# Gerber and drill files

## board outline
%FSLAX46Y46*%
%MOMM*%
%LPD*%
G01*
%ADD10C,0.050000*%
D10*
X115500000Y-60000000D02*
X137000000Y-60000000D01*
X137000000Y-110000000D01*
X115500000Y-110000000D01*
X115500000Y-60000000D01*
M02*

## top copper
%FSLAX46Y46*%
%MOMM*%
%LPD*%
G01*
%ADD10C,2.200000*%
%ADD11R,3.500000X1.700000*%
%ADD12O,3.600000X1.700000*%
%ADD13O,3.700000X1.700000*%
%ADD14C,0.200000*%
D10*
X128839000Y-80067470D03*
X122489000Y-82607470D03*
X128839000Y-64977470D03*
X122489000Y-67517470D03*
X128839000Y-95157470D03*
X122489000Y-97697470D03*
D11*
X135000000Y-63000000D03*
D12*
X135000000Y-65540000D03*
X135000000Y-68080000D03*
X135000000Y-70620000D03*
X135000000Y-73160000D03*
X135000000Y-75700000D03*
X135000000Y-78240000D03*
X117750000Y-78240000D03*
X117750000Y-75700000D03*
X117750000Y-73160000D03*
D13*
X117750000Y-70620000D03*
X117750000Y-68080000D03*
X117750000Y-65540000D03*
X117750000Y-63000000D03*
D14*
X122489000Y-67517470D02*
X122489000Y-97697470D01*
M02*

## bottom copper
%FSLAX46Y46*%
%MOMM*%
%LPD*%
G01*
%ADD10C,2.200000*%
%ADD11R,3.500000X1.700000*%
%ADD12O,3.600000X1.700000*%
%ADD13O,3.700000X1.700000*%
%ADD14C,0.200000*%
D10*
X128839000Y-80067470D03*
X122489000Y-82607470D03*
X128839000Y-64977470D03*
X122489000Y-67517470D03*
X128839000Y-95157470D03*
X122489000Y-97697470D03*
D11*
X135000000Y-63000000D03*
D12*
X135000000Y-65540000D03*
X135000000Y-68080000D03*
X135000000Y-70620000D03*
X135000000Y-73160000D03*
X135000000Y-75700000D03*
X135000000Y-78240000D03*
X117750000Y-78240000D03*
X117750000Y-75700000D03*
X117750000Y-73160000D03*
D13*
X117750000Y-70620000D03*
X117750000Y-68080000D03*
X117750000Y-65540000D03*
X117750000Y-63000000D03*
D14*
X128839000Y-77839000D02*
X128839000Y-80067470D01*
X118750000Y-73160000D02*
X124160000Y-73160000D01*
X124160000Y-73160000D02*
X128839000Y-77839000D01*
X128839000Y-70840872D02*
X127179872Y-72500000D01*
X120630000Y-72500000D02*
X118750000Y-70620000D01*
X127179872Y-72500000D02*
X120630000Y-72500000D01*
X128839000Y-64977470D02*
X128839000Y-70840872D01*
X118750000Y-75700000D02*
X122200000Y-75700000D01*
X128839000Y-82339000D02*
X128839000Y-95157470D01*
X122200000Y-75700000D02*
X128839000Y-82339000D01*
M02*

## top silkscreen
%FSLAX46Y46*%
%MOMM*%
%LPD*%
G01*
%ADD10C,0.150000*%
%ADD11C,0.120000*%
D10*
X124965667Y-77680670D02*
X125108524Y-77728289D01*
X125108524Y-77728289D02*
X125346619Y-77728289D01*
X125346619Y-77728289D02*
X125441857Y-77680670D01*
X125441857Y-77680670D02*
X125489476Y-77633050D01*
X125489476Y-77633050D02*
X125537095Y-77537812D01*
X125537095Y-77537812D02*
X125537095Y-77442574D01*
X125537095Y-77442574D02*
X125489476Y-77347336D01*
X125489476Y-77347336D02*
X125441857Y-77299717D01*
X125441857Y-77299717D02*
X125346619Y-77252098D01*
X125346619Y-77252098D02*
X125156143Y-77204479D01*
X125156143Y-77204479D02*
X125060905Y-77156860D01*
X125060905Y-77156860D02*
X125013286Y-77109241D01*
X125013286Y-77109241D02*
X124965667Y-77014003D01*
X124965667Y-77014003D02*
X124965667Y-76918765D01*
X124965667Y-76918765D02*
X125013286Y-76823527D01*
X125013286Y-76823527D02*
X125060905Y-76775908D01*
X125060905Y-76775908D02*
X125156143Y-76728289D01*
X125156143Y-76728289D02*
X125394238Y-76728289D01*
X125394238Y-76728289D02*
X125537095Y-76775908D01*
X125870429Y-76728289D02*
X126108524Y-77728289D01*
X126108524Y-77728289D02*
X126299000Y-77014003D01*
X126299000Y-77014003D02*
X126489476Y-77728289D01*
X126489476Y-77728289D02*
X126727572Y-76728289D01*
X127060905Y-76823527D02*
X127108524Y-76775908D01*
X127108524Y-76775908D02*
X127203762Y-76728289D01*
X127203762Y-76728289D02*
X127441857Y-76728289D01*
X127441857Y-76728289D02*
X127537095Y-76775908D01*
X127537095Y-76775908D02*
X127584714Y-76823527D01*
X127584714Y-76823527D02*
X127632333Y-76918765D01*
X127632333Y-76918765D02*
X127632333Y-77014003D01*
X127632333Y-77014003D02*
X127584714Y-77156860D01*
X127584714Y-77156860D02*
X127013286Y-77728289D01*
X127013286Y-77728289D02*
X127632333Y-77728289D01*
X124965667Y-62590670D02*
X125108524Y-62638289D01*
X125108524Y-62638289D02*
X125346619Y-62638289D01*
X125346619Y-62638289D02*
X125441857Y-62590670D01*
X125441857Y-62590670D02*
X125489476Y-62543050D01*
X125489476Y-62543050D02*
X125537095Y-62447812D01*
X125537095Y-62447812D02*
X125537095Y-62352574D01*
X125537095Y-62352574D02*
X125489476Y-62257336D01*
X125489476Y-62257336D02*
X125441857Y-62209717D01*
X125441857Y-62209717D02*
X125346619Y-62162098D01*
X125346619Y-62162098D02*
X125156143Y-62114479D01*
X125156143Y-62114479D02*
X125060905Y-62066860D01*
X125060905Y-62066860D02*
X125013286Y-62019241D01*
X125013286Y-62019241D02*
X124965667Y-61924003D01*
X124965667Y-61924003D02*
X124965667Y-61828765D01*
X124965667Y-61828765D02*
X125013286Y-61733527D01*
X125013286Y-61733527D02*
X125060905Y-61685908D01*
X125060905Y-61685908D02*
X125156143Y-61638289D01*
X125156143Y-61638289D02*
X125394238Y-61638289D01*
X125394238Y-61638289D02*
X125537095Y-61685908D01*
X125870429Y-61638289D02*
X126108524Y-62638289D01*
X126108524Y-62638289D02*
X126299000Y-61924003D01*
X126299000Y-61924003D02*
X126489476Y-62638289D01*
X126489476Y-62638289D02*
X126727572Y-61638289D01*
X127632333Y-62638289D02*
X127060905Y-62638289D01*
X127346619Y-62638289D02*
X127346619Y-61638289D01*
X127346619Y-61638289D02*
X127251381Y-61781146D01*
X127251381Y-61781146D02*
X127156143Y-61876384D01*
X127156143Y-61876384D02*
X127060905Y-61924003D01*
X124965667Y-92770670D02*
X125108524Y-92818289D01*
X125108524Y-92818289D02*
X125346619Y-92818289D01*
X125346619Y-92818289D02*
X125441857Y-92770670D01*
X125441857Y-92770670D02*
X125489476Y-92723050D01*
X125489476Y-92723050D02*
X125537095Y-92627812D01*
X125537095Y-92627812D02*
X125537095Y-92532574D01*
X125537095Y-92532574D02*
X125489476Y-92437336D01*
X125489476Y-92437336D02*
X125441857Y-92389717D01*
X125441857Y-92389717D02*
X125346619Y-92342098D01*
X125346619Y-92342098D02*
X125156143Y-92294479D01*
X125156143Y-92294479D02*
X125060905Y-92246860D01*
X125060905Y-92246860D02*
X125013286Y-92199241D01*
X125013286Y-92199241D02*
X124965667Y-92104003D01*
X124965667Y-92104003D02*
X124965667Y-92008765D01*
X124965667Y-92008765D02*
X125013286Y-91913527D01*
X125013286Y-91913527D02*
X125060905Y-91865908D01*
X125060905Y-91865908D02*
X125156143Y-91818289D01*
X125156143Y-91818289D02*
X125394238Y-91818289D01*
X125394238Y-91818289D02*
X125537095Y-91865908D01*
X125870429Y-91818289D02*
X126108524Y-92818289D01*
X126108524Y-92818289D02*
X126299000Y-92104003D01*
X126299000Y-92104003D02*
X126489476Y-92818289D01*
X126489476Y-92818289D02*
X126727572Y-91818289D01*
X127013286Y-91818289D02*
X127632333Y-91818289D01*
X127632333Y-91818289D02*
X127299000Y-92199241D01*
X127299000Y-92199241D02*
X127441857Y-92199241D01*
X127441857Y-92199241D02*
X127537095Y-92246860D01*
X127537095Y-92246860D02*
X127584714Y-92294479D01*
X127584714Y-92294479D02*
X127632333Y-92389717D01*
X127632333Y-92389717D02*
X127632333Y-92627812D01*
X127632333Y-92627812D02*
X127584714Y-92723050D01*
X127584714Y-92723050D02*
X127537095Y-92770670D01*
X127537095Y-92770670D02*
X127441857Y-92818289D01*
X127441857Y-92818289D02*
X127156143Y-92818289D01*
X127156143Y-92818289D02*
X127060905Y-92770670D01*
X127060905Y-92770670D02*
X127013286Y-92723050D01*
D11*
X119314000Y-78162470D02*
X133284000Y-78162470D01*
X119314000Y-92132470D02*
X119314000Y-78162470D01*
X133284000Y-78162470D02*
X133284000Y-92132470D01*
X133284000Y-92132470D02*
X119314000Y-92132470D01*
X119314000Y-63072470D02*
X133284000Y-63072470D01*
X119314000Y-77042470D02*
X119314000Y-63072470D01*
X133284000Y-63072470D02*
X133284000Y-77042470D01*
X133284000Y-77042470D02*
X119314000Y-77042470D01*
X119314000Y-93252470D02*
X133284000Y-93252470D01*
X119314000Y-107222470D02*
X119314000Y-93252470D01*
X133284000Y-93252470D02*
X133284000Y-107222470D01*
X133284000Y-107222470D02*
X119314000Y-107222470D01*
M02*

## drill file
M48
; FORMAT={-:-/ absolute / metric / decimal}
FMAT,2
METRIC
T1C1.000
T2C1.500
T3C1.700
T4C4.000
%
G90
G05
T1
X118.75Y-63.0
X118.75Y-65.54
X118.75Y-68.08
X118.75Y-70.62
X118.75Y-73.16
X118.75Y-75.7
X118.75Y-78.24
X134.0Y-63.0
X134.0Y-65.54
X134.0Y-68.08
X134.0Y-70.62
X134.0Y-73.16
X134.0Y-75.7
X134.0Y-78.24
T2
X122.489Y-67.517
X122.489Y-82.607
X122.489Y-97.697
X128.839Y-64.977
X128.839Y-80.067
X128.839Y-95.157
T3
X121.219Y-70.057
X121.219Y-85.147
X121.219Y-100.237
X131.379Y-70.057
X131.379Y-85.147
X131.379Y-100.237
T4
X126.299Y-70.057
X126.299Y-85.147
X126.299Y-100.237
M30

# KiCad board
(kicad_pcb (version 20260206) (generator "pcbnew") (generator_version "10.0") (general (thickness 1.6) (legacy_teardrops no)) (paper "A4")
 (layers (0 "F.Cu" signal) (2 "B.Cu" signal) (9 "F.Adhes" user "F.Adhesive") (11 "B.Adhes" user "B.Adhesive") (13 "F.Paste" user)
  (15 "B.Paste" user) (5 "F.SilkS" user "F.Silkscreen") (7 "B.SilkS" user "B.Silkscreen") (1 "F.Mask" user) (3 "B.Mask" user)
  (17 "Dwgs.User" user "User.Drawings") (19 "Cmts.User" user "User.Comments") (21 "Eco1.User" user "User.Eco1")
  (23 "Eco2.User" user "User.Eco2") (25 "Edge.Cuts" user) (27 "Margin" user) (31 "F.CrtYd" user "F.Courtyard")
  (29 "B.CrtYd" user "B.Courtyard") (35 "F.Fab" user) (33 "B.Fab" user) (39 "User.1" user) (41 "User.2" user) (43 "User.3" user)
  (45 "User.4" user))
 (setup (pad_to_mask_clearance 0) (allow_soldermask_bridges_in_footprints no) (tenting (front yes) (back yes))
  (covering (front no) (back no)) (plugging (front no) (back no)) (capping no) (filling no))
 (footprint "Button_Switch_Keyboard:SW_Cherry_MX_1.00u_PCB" (layer "F.Cu") (at 128.839 80.06747)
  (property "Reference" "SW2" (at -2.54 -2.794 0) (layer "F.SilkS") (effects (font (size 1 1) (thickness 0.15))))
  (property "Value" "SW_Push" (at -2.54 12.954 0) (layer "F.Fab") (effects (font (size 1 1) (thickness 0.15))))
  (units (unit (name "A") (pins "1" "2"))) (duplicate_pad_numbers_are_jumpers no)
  (fp_line (start -9.525 -1.905) (end 4.445 -1.905) (stroke (width 0.12) (type solid)) (layer "F.SilkS"))
  (fp_line (start -9.525 12.065) (end -9.525 -1.905) (stroke (width 0.12) (type solid)) (layer "F.SilkS"))
  (fp_line (start 4.445 -1.905) (end 4.445 12.065) (stroke (width 0.12) (type solid)) (layer "F.SilkS"))
  (fp_line (start 4.445 12.065) (end -9.525 12.065) (stroke (width 0.12) (type solid)) (layer "F.SilkS"))
  (pad "" np_thru_hole circle (at -7.62 5.08) (size 1.7 1.7) (drill 1.7) (layers "*.Cu" "*.Mask"))
  (pad "" np_thru_hole circle (at -2.54 5.08) (size 4 4) (drill 4) (layers "*.Cu" "*.Mask"))
  (pad "" np_thru_hole circle (at 2.54 5.08) (size 1.7 1.7) (drill 1.7) (layers "*.Cu" "*.Mask"))
  (pad "1" thru_hole circle (at 0 0) (size 2.2 2.2) (drill 1.5) (layers "*.Cu" "*.Mask") (remove_unused_layers no)
   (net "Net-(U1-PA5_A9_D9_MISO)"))
  (pad "2" thru_hole circle (at -6.35 2.54) (size 2.2 2.2) (drill 1.5) (layers "*.Cu" "*.Mask") (remove_unused_layers no) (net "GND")))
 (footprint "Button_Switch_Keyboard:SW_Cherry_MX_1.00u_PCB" (layer "F.Cu") (at 128.839 64.97747)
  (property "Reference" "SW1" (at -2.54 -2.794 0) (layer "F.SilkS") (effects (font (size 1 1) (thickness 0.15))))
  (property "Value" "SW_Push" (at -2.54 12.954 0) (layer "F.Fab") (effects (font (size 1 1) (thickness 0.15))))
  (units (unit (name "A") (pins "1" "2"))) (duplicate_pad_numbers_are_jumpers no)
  (fp_line (start -9.525 -1.905) (end 4.445 -1.905) (stroke (width 0.12) (type solid)) (layer "F.SilkS"))
  (fp_line (start -9.525 12.065) (end -9.525 -1.905) (stroke (width 0.12) (type solid)) (layer "F.SilkS"))
  (fp_line (start 4.445 -1.905) (end 4.445 12.065) (stroke (width 0.12) (type solid)) (layer "F.SilkS"))
  (fp_line (start 4.445 12.065) (end -9.525 12.065) (stroke (width 0.12) (type solid)) (layer "F.SilkS"))
  (pad "" np_thru_hole circle (at -7.62 5.08) (size 1.7 1.7) (drill 1.7) (layers "*.Cu" "*.Mask"))
  (pad "" np_thru_hole circle (at -2.54 5.08) (size 4 4) (drill 4) (layers "*.Cu" "*.Mask"))
  (pad "" np_thru_hole circle (at 2.54 5.08) (size 1.7 1.7) (drill 1.7) (layers "*.Cu" "*.Mask"))
  (pad "1" thru_hole circle (at 0 0) (size 2.2 2.2) (drill 1.5) (layers "*.Cu" "*.Mask") (remove_unused_layers no)
   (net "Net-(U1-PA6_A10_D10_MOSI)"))
  (pad "2" thru_hole circle (at -6.35 2.54) (size 2.2 2.2) (drill 1.5) (layers "*.Cu" "*.Mask") (remove_unused_layers no) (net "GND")))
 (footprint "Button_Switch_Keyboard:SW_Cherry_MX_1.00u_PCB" (layer "F.Cu") (at 128.839 95.15747)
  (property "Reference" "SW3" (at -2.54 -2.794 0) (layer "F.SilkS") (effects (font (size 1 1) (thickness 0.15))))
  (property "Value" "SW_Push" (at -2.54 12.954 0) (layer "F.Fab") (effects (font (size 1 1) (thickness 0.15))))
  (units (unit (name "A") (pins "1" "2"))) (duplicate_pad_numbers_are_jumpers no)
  (fp_line (start -9.525 -1.905) (end 4.445 -1.905) (stroke (width 0.12) (type solid)) (layer "F.SilkS"))
  (fp_line (start -9.525 12.065) (end -9.525 -1.905) (stroke (width 0.12) (type solid)) (layer "F.SilkS"))
  (fp_line (start 4.445 -1.905) (end 4.445 12.065) (stroke (width 0.12) (type solid)) (layer "F.SilkS"))
  (fp_line (start 4.445 12.065) (end -9.525 12.065) (stroke (width 0.12) (type solid)) (layer "F.SilkS"))
  (pad "" np_thru_hole circle (at -7.62 5.08) (size 1.7 1.7) (drill 1.7) (layers "*.Cu" "*.Mask"))
  (pad "" np_thru_hole circle (at -2.54 5.08) (size 4 4) (drill 4) (layers "*.Cu" "*.Mask"))
  (pad "" np_thru_hole circle (at 2.54 5.08) (size 1.7 1.7) (drill 1.7) (layers "*.Cu" "*.Mask"))
  (pad "1" thru_hole circle (at 0 0) (size 2.2 2.2) (drill 1.5) (layers "*.Cu" "*.Mask") (remove_unused_layers no)
   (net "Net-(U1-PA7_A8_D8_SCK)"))
  (pad "2" thru_hole circle (at -6.35 2.54) (size 2.2 2.2) (drill 1.5) (layers "*.Cu" "*.Mask") (remove_unused_layers no) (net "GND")))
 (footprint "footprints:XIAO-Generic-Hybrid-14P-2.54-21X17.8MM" (layer "B.Cu") (at 126.375 70.62 180)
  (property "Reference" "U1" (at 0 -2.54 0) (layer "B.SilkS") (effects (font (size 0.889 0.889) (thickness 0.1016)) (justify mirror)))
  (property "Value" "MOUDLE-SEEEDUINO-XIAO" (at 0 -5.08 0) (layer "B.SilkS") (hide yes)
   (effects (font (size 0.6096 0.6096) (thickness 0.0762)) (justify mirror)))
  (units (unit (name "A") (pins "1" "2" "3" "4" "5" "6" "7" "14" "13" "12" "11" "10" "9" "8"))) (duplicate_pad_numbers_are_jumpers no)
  (pad "1" thru_hole rect (at -7.625 7.62 180) (size 3.5 1.7) (drill 1 (offset -1 0)) (layers "*.Cu" "*.Mask") (remove_unused_layers no)
   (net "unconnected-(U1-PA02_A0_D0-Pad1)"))
  (pad "2" thru_hole oval (at -7.625 5.08 180) (size 3.6 1.7) (drill 1 (offset -1 0)) (layers "*.Cu" "*.Mask") (remove_unused_layers no)
   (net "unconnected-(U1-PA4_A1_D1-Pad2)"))
  (pad "3" thru_hole oval (at -7.625 2.54 180) (size 3.6 1.7) (drill 1 (offset -1 0)) (layers "*.Cu" "*.Mask") (remove_unused_layers no)
   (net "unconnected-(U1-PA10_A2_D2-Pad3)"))
  (pad "4" thru_hole oval (at -7.625 0 180) (size 3.6 1.7) (drill 1 (offset -1 0)) (layers "*.Cu" "*.Mask") (remove_unused_layers no)
   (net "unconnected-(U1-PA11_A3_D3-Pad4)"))
  (pad "5" thru_hole oval (at -7.625 -2.54 180) (size 3.6 1.7) (drill 1 (offset -1 0)) (layers "*.Cu" "*.Mask") (remove_unused_layers no)
   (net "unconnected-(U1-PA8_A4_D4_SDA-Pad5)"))
  (pad "6" thru_hole oval (at -7.625 -5.08) (size 3.6 1.7) (drill 1 (offset 1 0)) (layers "*.Cu" "*.Mask") (remove_unused_layers no)
   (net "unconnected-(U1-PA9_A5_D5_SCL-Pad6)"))
  (pad "7" thru_hole oval (at -7.625 -7.62 180) (size 3.6 1.7) (drill 1 (offset -1 0)) (layers "*.Cu" "*.Mask") (remove_unused_layers no)
   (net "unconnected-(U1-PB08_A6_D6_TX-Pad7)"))
  (pad "8" thru_hole oval (at 7.625 -7.62 180) (size 3.6 1.7) (drill 1 (offset 1 0)) (layers "*.Cu" "*.Mask") (remove_unused_layers no)
   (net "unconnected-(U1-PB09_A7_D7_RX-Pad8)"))
  (pad "9" thru_hole oval (at 7.625 -5.08 180) (size 3.6 1.7) (drill 1 (offset 1 0)) (layers "*.Cu" "*.Mask") (remove_unused_layers no)
   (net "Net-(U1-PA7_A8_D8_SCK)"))
  (pad "10" thru_hole oval (at 7.625 -2.54 180) (size 3.6 1.7) (drill 1 (offset 1 0)) (layers "*.Cu" "*.Mask") (remove_unused_layers no)
   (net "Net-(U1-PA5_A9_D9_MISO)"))
  (pad "11" thru_hole oval (at 7.625 0 180) (size 3.7 1.7) (drill 1 (offset 1 0)) (layers "*.Cu" "*.Mask") (remove_unused_layers no)
   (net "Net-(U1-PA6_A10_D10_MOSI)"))
  (pad "12" thru_hole oval (at 7.625 2.54 180) (size 3.7 1.7) (drill 1 (offset 1 0)) (layers "*.Cu" "*.Mask") (remove_unused_layers no)
   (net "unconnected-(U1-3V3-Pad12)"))
  (pad "13" thru_hole oval (at 7.625 5.08 180) (size 3.7 1.7) (drill 1 (offset 1 0)) (layers "*.Cu" "*.Mask") (remove_unused_layers no)
   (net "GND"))
  (pad "14" thru_hole oval (at 7.625 7.62 180) (size 3.7 1.7) (drill 1 (offset 1 0)) (layers "*.Cu" "*.Mask") (remove_unused_layers no)
   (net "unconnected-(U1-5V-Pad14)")))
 (gr_rect (start 115.5 60) (end 137 110) (stroke (width 0.05) (type default)) (fill no) (layer "Edge.Cuts"))
 (segment (start 128.839 77.839) (end 128.839 80.06747) (width 0.2) (layer "B.Cu") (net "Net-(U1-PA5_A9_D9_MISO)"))
 (segment (start 118.75 73.16) (end 124.16 73.16) (width 0.2) (layer "B.Cu") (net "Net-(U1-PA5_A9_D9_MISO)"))
 (segment (start 124.16 73.16) (end 128.839 77.839) (width 0.2) (layer "B.Cu") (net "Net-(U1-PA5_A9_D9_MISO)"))
 (segment (start 122.489 67.51747) (end 122.489 97.69747) (width 0.2) (layer "F.Cu") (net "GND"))
 (segment (start 128.839 70.840872) (end 127.179872 72.5) (width 0.2) (layer "B.Cu") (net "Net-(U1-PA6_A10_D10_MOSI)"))
 (segment (start 120.63 72.5) (end 118.75 70.62) (width 0.2) (layer "B.Cu") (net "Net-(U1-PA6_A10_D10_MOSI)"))
 (segment (start 127.179872 72.5) (end 120.63 72.5) (width 0.2) (layer "B.Cu") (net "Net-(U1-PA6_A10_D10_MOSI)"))
 (segment (start 128.839 64.97747) (end 128.839 70.840872) (width 0.2) (layer "B.Cu") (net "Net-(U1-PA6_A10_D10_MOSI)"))
 (segment (start 118.75 75.7) (end 122.2 75.7) (width 0.2) (layer "B.Cu") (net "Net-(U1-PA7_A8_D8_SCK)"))
 (segment (start 128.839 82.339) (end 128.839 95.15747) (width 0.2) (layer "B.Cu") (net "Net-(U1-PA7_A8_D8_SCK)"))
 (segment (start 122.2 75.7) (end 128.839 82.339) (width 0.2) (layer "B.Cu") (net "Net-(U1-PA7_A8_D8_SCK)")))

